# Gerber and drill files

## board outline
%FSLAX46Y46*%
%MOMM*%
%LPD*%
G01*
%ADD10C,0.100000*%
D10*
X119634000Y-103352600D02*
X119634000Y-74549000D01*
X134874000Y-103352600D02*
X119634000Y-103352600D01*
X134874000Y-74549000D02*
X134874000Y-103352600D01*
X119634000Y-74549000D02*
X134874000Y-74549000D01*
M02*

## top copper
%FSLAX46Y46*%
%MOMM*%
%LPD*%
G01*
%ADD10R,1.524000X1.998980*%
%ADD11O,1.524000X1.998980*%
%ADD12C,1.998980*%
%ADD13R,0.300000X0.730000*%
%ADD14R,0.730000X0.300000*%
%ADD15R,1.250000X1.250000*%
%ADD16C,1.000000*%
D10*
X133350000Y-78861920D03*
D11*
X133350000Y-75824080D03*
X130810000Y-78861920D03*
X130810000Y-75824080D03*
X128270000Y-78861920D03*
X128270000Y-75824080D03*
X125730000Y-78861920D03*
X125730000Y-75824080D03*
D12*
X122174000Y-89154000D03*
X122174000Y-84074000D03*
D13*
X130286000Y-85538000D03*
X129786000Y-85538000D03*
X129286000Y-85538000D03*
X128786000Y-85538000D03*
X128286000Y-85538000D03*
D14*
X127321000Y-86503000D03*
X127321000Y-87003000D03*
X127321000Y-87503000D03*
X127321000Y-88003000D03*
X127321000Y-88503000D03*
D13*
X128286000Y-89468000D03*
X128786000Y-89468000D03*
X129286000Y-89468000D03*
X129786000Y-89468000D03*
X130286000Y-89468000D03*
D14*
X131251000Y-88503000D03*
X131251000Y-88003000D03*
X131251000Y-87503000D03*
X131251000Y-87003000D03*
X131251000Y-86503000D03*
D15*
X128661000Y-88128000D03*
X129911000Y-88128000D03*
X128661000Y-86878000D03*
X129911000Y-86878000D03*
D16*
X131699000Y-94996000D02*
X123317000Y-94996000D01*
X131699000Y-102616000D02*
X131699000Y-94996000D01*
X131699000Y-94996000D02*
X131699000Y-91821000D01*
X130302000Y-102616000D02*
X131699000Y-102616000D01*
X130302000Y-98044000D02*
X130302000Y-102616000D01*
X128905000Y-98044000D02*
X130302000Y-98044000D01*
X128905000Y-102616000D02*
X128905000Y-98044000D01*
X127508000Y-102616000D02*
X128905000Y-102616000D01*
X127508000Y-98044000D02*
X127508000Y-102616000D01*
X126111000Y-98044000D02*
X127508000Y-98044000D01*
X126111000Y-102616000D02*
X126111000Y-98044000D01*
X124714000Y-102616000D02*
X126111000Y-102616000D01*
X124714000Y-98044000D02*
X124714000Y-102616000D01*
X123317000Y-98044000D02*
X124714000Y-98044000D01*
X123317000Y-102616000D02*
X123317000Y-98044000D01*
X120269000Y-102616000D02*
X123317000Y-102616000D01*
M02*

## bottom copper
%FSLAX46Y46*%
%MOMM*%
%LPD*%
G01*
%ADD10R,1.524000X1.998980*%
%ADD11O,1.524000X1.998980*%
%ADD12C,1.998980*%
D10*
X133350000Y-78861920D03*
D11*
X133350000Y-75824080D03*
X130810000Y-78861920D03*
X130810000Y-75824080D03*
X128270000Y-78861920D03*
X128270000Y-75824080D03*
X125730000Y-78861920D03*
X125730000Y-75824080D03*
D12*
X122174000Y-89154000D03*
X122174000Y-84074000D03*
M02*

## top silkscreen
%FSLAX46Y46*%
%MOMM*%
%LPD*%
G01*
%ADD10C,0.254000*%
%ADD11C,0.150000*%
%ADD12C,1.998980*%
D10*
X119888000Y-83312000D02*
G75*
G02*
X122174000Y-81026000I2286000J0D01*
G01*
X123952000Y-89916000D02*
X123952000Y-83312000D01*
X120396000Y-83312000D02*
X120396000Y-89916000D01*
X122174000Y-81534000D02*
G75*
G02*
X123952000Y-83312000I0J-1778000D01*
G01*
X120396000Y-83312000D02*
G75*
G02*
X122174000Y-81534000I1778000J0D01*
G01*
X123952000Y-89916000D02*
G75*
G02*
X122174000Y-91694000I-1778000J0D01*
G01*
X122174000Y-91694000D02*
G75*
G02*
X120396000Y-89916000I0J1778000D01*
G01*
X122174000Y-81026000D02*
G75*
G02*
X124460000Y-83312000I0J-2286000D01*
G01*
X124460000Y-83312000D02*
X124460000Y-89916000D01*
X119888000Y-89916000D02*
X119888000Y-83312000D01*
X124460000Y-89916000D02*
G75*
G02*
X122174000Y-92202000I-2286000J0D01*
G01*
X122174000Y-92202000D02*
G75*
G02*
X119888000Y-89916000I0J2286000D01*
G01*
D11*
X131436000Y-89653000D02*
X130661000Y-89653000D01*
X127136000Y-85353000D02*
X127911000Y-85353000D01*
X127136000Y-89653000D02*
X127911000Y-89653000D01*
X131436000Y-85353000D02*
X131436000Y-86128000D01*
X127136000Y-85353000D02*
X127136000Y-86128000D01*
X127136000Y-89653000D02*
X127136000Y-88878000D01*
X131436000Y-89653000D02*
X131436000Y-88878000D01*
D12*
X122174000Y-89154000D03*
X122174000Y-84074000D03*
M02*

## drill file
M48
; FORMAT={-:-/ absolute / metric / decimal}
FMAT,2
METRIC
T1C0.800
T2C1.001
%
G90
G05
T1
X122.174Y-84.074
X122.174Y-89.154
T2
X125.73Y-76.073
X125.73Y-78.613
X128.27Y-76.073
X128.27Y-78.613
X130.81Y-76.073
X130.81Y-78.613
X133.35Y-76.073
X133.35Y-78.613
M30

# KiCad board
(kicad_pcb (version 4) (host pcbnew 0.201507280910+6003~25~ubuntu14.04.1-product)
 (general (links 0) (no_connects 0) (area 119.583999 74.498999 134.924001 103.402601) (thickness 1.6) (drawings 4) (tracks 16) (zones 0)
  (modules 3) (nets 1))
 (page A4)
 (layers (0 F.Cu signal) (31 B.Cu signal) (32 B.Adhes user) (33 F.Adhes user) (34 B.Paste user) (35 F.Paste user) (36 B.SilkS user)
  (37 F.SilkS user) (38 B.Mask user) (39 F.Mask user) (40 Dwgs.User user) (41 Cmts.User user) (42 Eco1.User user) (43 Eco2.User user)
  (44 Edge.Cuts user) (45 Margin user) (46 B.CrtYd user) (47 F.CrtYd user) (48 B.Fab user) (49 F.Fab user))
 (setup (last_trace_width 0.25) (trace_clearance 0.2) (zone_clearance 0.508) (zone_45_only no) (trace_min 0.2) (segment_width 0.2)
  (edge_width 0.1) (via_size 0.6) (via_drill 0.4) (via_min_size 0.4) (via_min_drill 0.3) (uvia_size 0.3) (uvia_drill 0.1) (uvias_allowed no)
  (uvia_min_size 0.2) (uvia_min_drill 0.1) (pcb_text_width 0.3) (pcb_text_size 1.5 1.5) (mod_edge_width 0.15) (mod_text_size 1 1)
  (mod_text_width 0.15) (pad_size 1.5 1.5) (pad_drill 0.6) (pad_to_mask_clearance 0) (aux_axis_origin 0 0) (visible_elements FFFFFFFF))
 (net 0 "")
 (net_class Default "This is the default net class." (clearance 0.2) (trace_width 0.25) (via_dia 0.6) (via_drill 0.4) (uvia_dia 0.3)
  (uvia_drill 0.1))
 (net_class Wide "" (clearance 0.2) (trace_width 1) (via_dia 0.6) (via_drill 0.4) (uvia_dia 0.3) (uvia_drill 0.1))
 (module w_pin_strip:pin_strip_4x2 (layer B.Cu) (at 129.54 77.343 180)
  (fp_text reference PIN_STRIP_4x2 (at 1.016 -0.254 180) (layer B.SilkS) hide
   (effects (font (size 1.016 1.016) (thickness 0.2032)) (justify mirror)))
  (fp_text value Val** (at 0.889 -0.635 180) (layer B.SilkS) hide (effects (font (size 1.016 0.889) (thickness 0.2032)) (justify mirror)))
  (pad 1 thru_hole rect (at -3.81 -1.27 180) (size 1.524 1.99898) (drill 1.00076 (offset 0 -0.24892)) (layers *.Cu *.Mask B.SilkS))
  (pad 2 thru_hole oval (at -3.81 1.27 180) (size 1.524 1.99898) (drill 1.00076 (offset 0 0.24892)) (layers *.Cu *.Mask B.SilkS))
  (pad 3 thru_hole oval (at -1.27 -1.27 180) (size 1.524 1.99898) (drill 1.00076 (offset 0 -0.24892)) (layers *.Cu *.Mask B.SilkS))
  (pad 4 thru_hole oval (at -1.27 1.27 180) (size 1.524 1.99898) (drill 1.00076 (offset 0 0.24892)) (layers *.Cu *.Mask B.SilkS))
  (pad 5 thru_hole oval (at 1.27 -1.27 180) (size 1.524 1.99898) (drill 1.00076 (offset 0 -0.24892)) (layers *.Cu *.Mask B.SilkS))
  (pad 6 thru_hole oval (at 1.27 1.27 180) (size 1.524 1.99898) (drill 1.00076 (offset 0 0.24892)) (layers *.Cu *.Mask B.SilkS))
  (pad 7 thru_hole oval (at 3.81 -1.27 180) (size 1.524 1.99898) (drill 1.00076 (offset 0 -0.24892)) (layers *.Cu *.Mask B.SilkS))
  (pad 8 thru_hole oval (at 3.81 1.27 180) (size 1.524 1.99898) (drill 1.00076 (offset 0 0.24892)) (layers *.Cu *.Mask B.SilkS)))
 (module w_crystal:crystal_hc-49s (layer F.Cu) (at 122.174 86.614 90) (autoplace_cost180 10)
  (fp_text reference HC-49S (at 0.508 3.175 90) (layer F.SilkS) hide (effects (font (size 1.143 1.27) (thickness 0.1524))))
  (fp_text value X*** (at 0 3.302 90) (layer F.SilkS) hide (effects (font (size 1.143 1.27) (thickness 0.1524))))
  (fp_arc (start 3.302 0) (end 3.302 -2.286) (angle 90) (layer F.SilkS) (width 0.254))
  (fp_line (start -3.302 1.778) (end 3.302 1.778) (layer F.SilkS) (width 0.254))
  (fp_line (start 3.302 -1.778) (end -3.302 -1.778) (layer F.SilkS) (width 0.254))
  (fp_arc (start 3.302 0) (end 5.08 0) (angle 90) (layer F.SilkS) (width 0.254))
  (fp_arc (start 3.302 0) (end 3.302 -1.778) (angle 90) (layer F.SilkS) (width 0.254))
  (fp_arc (start -3.302 0) (end -3.302 1.778) (angle 90) (layer F.SilkS) (width 0.254))
  (fp_arc (start -3.302 0) (end -5.08 0) (angle 90) (layer F.SilkS) (width 0.254))
  (fp_arc (start 3.302 0) (end 5.588 0) (angle 90) (layer F.SilkS) (width 0.254))
  (fp_line (start 3.302 2.286) (end -3.302 2.286) (layer F.SilkS) (width 0.254))
  (fp_line (start -3.302 -2.286) (end 3.302 -2.286) (layer F.SilkS) (width 0.254))
  (fp_arc (start -3.302 0) (end -3.302 2.286) (angle 90) (layer F.SilkS) (width 0.254))
  (fp_arc (start -3.302 0) (end -5.588 0) (angle 90) (layer F.SilkS) (width 0.254))
  (pad 1 thru_hole circle (at -2.54 0 90) (size 1.99898 1.99898) (drill 0.8001) (layers *.Cu *.Mask F.SilkS))
  (pad 2 thru_hole circle (at 2.54 0 90) (size 1.99898 1.99898) (drill 0.8001) (layers *.Cu *.Mask F.SilkS)))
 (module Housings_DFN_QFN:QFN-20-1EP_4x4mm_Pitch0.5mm (layer F.Cu) (at 129.286 87.503 270)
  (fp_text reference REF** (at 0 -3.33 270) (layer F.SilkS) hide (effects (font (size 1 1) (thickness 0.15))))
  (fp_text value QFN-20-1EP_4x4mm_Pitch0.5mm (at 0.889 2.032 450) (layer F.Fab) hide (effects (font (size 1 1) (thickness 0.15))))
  (fp_line (start 2.15 -2.15) (end 2.15 -1.375) (layer F.SilkS) (width 0.15))
  (fp_line (start -2.15 2.15) (end -2.15 1.375) (layer F.SilkS) (width 0.15))
  (fp_line (start 2.15 2.15) (end 2.15 1.375) (layer F.SilkS) (width 0.15))
  (fp_line (start -2.15 -2.15) (end -1.375 -2.15) (layer F.SilkS) (width 0.15))
  (fp_line (start -2.15 2.15) (end -1.375 2.15) (layer F.SilkS) (width 0.15))
  (fp_line (start 2.15 2.15) (end 1.375 2.15) (layer F.SilkS) (width 0.15))
  (fp_line (start 2.15 -2.15) (end 1.375 -2.15) (layer F.SilkS) (width 0.15))
  (pad 1 smd rect (at -1.965 -1 270) (size 0.73 0.3) (layers F.Cu F.Paste F.Mask))
  (pad 2 smd rect (at -1.965 -0.5 270) (size 0.73 0.3) (layers F.Cu F.Paste F.Mask))
  (pad 3 smd rect (at -1.965 0 270) (size 0.73 0.3) (layers F.Cu F.Paste F.Mask))
  (pad 4 smd rect (at -1.965 0.5 270) (size 0.73 0.3) (layers F.Cu F.Paste F.Mask))
  (pad 5 smd rect (at -1.965 1 270) (size 0.73 0.3) (layers F.Cu F.Paste F.Mask))
  (pad 6 smd rect (at -1 1.965) (size 0.73 0.3) (layers F.Cu F.Paste F.Mask))
  (pad 7 smd rect (at -0.5 1.965) (size 0.73 0.3) (layers F.Cu F.Paste F.Mask))
  (pad 8 smd rect (at 0 1.965) (size 0.73 0.3) (layers F.Cu F.Paste F.Mask))
  (pad 9 smd rect (at 0.5 1.965) (size 0.73 0.3) (layers F.Cu F.Paste F.Mask))
  (pad 10 smd rect (at 1 1.965) (size 0.73 0.3) (layers F.Cu F.Paste F.Mask))
  (pad 11 smd rect (at 1.965 1 270) (size 0.73 0.3) (layers F.Cu F.Paste F.Mask))
  (pad 12 smd rect (at 1.965 0.5 270) (size 0.73 0.3) (layers F.Cu F.Paste F.Mask))
  (pad 13 smd rect (at 1.965 0 270) (size 0.73 0.3) (layers F.Cu F.Paste F.Mask))
  (pad 14 smd rect (at 1.965 -0.5 270) (size 0.73 0.3) (layers F.Cu F.Paste F.Mask))
  (pad 15 smd rect (at 1.965 -1 270) (size 0.73 0.3) (layers F.Cu F.Paste F.Mask))
  (pad 16 smd rect (at 1 -1.965) (size 0.73 0.3) (layers F.Cu F.Paste F.Mask))
  (pad 17 smd rect (at 0.5 -1.965) (size 0.73 0.3) (layers F.Cu F.Paste F.Mask))
  (pad 18 smd rect (at 0 -1.965) (size 0.73 0.3) (layers F.Cu F.Paste F.Mask))
  (pad 19 smd rect (at -0.5 -1.965) (size 0.73 0.3) (layers F.Cu F.Paste F.Mask))
  (pad 20 smd rect (at -1 -1.965) (size 0.73 0.3) (layers F.Cu F.Paste F.Mask))
  (pad 21 smd rect (at 0.625 0.625 270) (size 1.25 1.25) (layers F.Cu F.Paste F.Mask) (solder_paste_margin_ratio -0.2))
  (pad 21 smd rect (at 0.625 -0.625 270) (size 1.25 1.25) (layers F.Cu F.Paste F.Mask) (solder_paste_margin_ratio -0.2))
  (pad 21 smd rect (at -0.625 0.625 270) (size 1.25 1.25) (layers F.Cu F.Paste F.Mask) (solder_paste_margin_ratio -0.2))
  (pad 21 smd rect (at -0.625 -0.625 270) (size 1.25 1.25) (layers F.Cu F.Paste F.Mask) (solder_paste_margin_ratio -0.2)))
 (gr_line (start 119.634 103.3526) (end 119.634 74.549) (angle 90) (layer Edge.Cuts) (width 0.1))
 (gr_line (start 134.874 103.3526) (end 119.634 103.3526) (angle 90) (layer Edge.Cuts) (width 0.1))
 (gr_line (start 134.874 74.549) (end 134.874 103.3526) (angle 90) (layer Edge.Cuts) (width 0.1))
 (gr_line (start 119.634 74.549) (end 134.874 74.549) (angle 90) (layer Edge.Cuts) (width 0.1))
 (segment (start 131.699 94.996) (end 123.317 94.996) (width 1) (layer F.Cu) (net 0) (status 40000))
 (segment (start 131.699 102.616) (end 131.699 94.996) (width 1) (layer F.Cu) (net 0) (status 40000))
 (segment (start 131.699 94.996) (end 131.699 91.821) (width 1) (layer F.Cu) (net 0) (status 40000))
 (segment (start 130.302 102.616) (end 131.699 102.616) (width 1) (layer F.Cu) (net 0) (status 40000))
 (segment (start 130.302 98.044) (end 130.302 102.616) (width 1) (layer F.Cu) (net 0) (status 40000))
 (segment (start 128.905 98.044) (end 130.302 98.044) (width 1) (layer F.Cu) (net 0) (status 40000))
 (segment (start 128.905 102.616) (end 128.905 98.044) (width 1) (layer F.Cu) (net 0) (status 40000))
 (segment (start 127.508 102.616) (end 128.905 102.616) (width 1) (layer F.Cu) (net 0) (status 40000))
 (segment (start 127.508 98.044) (end 127.508 102.616) (width 1) (layer F.Cu) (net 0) (status 40000))
 (segment (start 126.111 98.044) (end 127.508 98.044) (width 1) (layer F.Cu) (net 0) (status 40000))
 (segment (start 126.111 102.616) (end 126.111 98.044) (width 1) (layer F.Cu) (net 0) (status 40000))
 (segment (start 124.714 102.616) (end 126.111 102.616) (width 1) (layer F.Cu) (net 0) (status 40000))
 (segment (start 124.714 98.044) (end 124.714 102.616) (width 1) (layer F.Cu) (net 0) (status 40000))
 (segment (start 123.317 98.044) (end 124.714 98.044) (width 1) (layer F.Cu) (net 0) (status 40000))
 (segment (start 123.317 102.616) (end 123.317 98.044) (width 1) (layer F.Cu) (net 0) (status 40000))
 (segment (start 120.269 102.616) (end 123.317 102.616) (width 1) (layer F.Cu) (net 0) (status 40000))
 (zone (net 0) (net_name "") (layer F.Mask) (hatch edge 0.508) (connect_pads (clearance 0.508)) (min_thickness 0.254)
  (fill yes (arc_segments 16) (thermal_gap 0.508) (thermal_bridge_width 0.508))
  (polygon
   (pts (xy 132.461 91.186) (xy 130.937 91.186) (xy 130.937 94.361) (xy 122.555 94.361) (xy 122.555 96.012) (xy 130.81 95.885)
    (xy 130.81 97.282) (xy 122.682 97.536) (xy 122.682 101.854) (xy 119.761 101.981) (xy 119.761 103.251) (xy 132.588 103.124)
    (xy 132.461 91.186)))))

